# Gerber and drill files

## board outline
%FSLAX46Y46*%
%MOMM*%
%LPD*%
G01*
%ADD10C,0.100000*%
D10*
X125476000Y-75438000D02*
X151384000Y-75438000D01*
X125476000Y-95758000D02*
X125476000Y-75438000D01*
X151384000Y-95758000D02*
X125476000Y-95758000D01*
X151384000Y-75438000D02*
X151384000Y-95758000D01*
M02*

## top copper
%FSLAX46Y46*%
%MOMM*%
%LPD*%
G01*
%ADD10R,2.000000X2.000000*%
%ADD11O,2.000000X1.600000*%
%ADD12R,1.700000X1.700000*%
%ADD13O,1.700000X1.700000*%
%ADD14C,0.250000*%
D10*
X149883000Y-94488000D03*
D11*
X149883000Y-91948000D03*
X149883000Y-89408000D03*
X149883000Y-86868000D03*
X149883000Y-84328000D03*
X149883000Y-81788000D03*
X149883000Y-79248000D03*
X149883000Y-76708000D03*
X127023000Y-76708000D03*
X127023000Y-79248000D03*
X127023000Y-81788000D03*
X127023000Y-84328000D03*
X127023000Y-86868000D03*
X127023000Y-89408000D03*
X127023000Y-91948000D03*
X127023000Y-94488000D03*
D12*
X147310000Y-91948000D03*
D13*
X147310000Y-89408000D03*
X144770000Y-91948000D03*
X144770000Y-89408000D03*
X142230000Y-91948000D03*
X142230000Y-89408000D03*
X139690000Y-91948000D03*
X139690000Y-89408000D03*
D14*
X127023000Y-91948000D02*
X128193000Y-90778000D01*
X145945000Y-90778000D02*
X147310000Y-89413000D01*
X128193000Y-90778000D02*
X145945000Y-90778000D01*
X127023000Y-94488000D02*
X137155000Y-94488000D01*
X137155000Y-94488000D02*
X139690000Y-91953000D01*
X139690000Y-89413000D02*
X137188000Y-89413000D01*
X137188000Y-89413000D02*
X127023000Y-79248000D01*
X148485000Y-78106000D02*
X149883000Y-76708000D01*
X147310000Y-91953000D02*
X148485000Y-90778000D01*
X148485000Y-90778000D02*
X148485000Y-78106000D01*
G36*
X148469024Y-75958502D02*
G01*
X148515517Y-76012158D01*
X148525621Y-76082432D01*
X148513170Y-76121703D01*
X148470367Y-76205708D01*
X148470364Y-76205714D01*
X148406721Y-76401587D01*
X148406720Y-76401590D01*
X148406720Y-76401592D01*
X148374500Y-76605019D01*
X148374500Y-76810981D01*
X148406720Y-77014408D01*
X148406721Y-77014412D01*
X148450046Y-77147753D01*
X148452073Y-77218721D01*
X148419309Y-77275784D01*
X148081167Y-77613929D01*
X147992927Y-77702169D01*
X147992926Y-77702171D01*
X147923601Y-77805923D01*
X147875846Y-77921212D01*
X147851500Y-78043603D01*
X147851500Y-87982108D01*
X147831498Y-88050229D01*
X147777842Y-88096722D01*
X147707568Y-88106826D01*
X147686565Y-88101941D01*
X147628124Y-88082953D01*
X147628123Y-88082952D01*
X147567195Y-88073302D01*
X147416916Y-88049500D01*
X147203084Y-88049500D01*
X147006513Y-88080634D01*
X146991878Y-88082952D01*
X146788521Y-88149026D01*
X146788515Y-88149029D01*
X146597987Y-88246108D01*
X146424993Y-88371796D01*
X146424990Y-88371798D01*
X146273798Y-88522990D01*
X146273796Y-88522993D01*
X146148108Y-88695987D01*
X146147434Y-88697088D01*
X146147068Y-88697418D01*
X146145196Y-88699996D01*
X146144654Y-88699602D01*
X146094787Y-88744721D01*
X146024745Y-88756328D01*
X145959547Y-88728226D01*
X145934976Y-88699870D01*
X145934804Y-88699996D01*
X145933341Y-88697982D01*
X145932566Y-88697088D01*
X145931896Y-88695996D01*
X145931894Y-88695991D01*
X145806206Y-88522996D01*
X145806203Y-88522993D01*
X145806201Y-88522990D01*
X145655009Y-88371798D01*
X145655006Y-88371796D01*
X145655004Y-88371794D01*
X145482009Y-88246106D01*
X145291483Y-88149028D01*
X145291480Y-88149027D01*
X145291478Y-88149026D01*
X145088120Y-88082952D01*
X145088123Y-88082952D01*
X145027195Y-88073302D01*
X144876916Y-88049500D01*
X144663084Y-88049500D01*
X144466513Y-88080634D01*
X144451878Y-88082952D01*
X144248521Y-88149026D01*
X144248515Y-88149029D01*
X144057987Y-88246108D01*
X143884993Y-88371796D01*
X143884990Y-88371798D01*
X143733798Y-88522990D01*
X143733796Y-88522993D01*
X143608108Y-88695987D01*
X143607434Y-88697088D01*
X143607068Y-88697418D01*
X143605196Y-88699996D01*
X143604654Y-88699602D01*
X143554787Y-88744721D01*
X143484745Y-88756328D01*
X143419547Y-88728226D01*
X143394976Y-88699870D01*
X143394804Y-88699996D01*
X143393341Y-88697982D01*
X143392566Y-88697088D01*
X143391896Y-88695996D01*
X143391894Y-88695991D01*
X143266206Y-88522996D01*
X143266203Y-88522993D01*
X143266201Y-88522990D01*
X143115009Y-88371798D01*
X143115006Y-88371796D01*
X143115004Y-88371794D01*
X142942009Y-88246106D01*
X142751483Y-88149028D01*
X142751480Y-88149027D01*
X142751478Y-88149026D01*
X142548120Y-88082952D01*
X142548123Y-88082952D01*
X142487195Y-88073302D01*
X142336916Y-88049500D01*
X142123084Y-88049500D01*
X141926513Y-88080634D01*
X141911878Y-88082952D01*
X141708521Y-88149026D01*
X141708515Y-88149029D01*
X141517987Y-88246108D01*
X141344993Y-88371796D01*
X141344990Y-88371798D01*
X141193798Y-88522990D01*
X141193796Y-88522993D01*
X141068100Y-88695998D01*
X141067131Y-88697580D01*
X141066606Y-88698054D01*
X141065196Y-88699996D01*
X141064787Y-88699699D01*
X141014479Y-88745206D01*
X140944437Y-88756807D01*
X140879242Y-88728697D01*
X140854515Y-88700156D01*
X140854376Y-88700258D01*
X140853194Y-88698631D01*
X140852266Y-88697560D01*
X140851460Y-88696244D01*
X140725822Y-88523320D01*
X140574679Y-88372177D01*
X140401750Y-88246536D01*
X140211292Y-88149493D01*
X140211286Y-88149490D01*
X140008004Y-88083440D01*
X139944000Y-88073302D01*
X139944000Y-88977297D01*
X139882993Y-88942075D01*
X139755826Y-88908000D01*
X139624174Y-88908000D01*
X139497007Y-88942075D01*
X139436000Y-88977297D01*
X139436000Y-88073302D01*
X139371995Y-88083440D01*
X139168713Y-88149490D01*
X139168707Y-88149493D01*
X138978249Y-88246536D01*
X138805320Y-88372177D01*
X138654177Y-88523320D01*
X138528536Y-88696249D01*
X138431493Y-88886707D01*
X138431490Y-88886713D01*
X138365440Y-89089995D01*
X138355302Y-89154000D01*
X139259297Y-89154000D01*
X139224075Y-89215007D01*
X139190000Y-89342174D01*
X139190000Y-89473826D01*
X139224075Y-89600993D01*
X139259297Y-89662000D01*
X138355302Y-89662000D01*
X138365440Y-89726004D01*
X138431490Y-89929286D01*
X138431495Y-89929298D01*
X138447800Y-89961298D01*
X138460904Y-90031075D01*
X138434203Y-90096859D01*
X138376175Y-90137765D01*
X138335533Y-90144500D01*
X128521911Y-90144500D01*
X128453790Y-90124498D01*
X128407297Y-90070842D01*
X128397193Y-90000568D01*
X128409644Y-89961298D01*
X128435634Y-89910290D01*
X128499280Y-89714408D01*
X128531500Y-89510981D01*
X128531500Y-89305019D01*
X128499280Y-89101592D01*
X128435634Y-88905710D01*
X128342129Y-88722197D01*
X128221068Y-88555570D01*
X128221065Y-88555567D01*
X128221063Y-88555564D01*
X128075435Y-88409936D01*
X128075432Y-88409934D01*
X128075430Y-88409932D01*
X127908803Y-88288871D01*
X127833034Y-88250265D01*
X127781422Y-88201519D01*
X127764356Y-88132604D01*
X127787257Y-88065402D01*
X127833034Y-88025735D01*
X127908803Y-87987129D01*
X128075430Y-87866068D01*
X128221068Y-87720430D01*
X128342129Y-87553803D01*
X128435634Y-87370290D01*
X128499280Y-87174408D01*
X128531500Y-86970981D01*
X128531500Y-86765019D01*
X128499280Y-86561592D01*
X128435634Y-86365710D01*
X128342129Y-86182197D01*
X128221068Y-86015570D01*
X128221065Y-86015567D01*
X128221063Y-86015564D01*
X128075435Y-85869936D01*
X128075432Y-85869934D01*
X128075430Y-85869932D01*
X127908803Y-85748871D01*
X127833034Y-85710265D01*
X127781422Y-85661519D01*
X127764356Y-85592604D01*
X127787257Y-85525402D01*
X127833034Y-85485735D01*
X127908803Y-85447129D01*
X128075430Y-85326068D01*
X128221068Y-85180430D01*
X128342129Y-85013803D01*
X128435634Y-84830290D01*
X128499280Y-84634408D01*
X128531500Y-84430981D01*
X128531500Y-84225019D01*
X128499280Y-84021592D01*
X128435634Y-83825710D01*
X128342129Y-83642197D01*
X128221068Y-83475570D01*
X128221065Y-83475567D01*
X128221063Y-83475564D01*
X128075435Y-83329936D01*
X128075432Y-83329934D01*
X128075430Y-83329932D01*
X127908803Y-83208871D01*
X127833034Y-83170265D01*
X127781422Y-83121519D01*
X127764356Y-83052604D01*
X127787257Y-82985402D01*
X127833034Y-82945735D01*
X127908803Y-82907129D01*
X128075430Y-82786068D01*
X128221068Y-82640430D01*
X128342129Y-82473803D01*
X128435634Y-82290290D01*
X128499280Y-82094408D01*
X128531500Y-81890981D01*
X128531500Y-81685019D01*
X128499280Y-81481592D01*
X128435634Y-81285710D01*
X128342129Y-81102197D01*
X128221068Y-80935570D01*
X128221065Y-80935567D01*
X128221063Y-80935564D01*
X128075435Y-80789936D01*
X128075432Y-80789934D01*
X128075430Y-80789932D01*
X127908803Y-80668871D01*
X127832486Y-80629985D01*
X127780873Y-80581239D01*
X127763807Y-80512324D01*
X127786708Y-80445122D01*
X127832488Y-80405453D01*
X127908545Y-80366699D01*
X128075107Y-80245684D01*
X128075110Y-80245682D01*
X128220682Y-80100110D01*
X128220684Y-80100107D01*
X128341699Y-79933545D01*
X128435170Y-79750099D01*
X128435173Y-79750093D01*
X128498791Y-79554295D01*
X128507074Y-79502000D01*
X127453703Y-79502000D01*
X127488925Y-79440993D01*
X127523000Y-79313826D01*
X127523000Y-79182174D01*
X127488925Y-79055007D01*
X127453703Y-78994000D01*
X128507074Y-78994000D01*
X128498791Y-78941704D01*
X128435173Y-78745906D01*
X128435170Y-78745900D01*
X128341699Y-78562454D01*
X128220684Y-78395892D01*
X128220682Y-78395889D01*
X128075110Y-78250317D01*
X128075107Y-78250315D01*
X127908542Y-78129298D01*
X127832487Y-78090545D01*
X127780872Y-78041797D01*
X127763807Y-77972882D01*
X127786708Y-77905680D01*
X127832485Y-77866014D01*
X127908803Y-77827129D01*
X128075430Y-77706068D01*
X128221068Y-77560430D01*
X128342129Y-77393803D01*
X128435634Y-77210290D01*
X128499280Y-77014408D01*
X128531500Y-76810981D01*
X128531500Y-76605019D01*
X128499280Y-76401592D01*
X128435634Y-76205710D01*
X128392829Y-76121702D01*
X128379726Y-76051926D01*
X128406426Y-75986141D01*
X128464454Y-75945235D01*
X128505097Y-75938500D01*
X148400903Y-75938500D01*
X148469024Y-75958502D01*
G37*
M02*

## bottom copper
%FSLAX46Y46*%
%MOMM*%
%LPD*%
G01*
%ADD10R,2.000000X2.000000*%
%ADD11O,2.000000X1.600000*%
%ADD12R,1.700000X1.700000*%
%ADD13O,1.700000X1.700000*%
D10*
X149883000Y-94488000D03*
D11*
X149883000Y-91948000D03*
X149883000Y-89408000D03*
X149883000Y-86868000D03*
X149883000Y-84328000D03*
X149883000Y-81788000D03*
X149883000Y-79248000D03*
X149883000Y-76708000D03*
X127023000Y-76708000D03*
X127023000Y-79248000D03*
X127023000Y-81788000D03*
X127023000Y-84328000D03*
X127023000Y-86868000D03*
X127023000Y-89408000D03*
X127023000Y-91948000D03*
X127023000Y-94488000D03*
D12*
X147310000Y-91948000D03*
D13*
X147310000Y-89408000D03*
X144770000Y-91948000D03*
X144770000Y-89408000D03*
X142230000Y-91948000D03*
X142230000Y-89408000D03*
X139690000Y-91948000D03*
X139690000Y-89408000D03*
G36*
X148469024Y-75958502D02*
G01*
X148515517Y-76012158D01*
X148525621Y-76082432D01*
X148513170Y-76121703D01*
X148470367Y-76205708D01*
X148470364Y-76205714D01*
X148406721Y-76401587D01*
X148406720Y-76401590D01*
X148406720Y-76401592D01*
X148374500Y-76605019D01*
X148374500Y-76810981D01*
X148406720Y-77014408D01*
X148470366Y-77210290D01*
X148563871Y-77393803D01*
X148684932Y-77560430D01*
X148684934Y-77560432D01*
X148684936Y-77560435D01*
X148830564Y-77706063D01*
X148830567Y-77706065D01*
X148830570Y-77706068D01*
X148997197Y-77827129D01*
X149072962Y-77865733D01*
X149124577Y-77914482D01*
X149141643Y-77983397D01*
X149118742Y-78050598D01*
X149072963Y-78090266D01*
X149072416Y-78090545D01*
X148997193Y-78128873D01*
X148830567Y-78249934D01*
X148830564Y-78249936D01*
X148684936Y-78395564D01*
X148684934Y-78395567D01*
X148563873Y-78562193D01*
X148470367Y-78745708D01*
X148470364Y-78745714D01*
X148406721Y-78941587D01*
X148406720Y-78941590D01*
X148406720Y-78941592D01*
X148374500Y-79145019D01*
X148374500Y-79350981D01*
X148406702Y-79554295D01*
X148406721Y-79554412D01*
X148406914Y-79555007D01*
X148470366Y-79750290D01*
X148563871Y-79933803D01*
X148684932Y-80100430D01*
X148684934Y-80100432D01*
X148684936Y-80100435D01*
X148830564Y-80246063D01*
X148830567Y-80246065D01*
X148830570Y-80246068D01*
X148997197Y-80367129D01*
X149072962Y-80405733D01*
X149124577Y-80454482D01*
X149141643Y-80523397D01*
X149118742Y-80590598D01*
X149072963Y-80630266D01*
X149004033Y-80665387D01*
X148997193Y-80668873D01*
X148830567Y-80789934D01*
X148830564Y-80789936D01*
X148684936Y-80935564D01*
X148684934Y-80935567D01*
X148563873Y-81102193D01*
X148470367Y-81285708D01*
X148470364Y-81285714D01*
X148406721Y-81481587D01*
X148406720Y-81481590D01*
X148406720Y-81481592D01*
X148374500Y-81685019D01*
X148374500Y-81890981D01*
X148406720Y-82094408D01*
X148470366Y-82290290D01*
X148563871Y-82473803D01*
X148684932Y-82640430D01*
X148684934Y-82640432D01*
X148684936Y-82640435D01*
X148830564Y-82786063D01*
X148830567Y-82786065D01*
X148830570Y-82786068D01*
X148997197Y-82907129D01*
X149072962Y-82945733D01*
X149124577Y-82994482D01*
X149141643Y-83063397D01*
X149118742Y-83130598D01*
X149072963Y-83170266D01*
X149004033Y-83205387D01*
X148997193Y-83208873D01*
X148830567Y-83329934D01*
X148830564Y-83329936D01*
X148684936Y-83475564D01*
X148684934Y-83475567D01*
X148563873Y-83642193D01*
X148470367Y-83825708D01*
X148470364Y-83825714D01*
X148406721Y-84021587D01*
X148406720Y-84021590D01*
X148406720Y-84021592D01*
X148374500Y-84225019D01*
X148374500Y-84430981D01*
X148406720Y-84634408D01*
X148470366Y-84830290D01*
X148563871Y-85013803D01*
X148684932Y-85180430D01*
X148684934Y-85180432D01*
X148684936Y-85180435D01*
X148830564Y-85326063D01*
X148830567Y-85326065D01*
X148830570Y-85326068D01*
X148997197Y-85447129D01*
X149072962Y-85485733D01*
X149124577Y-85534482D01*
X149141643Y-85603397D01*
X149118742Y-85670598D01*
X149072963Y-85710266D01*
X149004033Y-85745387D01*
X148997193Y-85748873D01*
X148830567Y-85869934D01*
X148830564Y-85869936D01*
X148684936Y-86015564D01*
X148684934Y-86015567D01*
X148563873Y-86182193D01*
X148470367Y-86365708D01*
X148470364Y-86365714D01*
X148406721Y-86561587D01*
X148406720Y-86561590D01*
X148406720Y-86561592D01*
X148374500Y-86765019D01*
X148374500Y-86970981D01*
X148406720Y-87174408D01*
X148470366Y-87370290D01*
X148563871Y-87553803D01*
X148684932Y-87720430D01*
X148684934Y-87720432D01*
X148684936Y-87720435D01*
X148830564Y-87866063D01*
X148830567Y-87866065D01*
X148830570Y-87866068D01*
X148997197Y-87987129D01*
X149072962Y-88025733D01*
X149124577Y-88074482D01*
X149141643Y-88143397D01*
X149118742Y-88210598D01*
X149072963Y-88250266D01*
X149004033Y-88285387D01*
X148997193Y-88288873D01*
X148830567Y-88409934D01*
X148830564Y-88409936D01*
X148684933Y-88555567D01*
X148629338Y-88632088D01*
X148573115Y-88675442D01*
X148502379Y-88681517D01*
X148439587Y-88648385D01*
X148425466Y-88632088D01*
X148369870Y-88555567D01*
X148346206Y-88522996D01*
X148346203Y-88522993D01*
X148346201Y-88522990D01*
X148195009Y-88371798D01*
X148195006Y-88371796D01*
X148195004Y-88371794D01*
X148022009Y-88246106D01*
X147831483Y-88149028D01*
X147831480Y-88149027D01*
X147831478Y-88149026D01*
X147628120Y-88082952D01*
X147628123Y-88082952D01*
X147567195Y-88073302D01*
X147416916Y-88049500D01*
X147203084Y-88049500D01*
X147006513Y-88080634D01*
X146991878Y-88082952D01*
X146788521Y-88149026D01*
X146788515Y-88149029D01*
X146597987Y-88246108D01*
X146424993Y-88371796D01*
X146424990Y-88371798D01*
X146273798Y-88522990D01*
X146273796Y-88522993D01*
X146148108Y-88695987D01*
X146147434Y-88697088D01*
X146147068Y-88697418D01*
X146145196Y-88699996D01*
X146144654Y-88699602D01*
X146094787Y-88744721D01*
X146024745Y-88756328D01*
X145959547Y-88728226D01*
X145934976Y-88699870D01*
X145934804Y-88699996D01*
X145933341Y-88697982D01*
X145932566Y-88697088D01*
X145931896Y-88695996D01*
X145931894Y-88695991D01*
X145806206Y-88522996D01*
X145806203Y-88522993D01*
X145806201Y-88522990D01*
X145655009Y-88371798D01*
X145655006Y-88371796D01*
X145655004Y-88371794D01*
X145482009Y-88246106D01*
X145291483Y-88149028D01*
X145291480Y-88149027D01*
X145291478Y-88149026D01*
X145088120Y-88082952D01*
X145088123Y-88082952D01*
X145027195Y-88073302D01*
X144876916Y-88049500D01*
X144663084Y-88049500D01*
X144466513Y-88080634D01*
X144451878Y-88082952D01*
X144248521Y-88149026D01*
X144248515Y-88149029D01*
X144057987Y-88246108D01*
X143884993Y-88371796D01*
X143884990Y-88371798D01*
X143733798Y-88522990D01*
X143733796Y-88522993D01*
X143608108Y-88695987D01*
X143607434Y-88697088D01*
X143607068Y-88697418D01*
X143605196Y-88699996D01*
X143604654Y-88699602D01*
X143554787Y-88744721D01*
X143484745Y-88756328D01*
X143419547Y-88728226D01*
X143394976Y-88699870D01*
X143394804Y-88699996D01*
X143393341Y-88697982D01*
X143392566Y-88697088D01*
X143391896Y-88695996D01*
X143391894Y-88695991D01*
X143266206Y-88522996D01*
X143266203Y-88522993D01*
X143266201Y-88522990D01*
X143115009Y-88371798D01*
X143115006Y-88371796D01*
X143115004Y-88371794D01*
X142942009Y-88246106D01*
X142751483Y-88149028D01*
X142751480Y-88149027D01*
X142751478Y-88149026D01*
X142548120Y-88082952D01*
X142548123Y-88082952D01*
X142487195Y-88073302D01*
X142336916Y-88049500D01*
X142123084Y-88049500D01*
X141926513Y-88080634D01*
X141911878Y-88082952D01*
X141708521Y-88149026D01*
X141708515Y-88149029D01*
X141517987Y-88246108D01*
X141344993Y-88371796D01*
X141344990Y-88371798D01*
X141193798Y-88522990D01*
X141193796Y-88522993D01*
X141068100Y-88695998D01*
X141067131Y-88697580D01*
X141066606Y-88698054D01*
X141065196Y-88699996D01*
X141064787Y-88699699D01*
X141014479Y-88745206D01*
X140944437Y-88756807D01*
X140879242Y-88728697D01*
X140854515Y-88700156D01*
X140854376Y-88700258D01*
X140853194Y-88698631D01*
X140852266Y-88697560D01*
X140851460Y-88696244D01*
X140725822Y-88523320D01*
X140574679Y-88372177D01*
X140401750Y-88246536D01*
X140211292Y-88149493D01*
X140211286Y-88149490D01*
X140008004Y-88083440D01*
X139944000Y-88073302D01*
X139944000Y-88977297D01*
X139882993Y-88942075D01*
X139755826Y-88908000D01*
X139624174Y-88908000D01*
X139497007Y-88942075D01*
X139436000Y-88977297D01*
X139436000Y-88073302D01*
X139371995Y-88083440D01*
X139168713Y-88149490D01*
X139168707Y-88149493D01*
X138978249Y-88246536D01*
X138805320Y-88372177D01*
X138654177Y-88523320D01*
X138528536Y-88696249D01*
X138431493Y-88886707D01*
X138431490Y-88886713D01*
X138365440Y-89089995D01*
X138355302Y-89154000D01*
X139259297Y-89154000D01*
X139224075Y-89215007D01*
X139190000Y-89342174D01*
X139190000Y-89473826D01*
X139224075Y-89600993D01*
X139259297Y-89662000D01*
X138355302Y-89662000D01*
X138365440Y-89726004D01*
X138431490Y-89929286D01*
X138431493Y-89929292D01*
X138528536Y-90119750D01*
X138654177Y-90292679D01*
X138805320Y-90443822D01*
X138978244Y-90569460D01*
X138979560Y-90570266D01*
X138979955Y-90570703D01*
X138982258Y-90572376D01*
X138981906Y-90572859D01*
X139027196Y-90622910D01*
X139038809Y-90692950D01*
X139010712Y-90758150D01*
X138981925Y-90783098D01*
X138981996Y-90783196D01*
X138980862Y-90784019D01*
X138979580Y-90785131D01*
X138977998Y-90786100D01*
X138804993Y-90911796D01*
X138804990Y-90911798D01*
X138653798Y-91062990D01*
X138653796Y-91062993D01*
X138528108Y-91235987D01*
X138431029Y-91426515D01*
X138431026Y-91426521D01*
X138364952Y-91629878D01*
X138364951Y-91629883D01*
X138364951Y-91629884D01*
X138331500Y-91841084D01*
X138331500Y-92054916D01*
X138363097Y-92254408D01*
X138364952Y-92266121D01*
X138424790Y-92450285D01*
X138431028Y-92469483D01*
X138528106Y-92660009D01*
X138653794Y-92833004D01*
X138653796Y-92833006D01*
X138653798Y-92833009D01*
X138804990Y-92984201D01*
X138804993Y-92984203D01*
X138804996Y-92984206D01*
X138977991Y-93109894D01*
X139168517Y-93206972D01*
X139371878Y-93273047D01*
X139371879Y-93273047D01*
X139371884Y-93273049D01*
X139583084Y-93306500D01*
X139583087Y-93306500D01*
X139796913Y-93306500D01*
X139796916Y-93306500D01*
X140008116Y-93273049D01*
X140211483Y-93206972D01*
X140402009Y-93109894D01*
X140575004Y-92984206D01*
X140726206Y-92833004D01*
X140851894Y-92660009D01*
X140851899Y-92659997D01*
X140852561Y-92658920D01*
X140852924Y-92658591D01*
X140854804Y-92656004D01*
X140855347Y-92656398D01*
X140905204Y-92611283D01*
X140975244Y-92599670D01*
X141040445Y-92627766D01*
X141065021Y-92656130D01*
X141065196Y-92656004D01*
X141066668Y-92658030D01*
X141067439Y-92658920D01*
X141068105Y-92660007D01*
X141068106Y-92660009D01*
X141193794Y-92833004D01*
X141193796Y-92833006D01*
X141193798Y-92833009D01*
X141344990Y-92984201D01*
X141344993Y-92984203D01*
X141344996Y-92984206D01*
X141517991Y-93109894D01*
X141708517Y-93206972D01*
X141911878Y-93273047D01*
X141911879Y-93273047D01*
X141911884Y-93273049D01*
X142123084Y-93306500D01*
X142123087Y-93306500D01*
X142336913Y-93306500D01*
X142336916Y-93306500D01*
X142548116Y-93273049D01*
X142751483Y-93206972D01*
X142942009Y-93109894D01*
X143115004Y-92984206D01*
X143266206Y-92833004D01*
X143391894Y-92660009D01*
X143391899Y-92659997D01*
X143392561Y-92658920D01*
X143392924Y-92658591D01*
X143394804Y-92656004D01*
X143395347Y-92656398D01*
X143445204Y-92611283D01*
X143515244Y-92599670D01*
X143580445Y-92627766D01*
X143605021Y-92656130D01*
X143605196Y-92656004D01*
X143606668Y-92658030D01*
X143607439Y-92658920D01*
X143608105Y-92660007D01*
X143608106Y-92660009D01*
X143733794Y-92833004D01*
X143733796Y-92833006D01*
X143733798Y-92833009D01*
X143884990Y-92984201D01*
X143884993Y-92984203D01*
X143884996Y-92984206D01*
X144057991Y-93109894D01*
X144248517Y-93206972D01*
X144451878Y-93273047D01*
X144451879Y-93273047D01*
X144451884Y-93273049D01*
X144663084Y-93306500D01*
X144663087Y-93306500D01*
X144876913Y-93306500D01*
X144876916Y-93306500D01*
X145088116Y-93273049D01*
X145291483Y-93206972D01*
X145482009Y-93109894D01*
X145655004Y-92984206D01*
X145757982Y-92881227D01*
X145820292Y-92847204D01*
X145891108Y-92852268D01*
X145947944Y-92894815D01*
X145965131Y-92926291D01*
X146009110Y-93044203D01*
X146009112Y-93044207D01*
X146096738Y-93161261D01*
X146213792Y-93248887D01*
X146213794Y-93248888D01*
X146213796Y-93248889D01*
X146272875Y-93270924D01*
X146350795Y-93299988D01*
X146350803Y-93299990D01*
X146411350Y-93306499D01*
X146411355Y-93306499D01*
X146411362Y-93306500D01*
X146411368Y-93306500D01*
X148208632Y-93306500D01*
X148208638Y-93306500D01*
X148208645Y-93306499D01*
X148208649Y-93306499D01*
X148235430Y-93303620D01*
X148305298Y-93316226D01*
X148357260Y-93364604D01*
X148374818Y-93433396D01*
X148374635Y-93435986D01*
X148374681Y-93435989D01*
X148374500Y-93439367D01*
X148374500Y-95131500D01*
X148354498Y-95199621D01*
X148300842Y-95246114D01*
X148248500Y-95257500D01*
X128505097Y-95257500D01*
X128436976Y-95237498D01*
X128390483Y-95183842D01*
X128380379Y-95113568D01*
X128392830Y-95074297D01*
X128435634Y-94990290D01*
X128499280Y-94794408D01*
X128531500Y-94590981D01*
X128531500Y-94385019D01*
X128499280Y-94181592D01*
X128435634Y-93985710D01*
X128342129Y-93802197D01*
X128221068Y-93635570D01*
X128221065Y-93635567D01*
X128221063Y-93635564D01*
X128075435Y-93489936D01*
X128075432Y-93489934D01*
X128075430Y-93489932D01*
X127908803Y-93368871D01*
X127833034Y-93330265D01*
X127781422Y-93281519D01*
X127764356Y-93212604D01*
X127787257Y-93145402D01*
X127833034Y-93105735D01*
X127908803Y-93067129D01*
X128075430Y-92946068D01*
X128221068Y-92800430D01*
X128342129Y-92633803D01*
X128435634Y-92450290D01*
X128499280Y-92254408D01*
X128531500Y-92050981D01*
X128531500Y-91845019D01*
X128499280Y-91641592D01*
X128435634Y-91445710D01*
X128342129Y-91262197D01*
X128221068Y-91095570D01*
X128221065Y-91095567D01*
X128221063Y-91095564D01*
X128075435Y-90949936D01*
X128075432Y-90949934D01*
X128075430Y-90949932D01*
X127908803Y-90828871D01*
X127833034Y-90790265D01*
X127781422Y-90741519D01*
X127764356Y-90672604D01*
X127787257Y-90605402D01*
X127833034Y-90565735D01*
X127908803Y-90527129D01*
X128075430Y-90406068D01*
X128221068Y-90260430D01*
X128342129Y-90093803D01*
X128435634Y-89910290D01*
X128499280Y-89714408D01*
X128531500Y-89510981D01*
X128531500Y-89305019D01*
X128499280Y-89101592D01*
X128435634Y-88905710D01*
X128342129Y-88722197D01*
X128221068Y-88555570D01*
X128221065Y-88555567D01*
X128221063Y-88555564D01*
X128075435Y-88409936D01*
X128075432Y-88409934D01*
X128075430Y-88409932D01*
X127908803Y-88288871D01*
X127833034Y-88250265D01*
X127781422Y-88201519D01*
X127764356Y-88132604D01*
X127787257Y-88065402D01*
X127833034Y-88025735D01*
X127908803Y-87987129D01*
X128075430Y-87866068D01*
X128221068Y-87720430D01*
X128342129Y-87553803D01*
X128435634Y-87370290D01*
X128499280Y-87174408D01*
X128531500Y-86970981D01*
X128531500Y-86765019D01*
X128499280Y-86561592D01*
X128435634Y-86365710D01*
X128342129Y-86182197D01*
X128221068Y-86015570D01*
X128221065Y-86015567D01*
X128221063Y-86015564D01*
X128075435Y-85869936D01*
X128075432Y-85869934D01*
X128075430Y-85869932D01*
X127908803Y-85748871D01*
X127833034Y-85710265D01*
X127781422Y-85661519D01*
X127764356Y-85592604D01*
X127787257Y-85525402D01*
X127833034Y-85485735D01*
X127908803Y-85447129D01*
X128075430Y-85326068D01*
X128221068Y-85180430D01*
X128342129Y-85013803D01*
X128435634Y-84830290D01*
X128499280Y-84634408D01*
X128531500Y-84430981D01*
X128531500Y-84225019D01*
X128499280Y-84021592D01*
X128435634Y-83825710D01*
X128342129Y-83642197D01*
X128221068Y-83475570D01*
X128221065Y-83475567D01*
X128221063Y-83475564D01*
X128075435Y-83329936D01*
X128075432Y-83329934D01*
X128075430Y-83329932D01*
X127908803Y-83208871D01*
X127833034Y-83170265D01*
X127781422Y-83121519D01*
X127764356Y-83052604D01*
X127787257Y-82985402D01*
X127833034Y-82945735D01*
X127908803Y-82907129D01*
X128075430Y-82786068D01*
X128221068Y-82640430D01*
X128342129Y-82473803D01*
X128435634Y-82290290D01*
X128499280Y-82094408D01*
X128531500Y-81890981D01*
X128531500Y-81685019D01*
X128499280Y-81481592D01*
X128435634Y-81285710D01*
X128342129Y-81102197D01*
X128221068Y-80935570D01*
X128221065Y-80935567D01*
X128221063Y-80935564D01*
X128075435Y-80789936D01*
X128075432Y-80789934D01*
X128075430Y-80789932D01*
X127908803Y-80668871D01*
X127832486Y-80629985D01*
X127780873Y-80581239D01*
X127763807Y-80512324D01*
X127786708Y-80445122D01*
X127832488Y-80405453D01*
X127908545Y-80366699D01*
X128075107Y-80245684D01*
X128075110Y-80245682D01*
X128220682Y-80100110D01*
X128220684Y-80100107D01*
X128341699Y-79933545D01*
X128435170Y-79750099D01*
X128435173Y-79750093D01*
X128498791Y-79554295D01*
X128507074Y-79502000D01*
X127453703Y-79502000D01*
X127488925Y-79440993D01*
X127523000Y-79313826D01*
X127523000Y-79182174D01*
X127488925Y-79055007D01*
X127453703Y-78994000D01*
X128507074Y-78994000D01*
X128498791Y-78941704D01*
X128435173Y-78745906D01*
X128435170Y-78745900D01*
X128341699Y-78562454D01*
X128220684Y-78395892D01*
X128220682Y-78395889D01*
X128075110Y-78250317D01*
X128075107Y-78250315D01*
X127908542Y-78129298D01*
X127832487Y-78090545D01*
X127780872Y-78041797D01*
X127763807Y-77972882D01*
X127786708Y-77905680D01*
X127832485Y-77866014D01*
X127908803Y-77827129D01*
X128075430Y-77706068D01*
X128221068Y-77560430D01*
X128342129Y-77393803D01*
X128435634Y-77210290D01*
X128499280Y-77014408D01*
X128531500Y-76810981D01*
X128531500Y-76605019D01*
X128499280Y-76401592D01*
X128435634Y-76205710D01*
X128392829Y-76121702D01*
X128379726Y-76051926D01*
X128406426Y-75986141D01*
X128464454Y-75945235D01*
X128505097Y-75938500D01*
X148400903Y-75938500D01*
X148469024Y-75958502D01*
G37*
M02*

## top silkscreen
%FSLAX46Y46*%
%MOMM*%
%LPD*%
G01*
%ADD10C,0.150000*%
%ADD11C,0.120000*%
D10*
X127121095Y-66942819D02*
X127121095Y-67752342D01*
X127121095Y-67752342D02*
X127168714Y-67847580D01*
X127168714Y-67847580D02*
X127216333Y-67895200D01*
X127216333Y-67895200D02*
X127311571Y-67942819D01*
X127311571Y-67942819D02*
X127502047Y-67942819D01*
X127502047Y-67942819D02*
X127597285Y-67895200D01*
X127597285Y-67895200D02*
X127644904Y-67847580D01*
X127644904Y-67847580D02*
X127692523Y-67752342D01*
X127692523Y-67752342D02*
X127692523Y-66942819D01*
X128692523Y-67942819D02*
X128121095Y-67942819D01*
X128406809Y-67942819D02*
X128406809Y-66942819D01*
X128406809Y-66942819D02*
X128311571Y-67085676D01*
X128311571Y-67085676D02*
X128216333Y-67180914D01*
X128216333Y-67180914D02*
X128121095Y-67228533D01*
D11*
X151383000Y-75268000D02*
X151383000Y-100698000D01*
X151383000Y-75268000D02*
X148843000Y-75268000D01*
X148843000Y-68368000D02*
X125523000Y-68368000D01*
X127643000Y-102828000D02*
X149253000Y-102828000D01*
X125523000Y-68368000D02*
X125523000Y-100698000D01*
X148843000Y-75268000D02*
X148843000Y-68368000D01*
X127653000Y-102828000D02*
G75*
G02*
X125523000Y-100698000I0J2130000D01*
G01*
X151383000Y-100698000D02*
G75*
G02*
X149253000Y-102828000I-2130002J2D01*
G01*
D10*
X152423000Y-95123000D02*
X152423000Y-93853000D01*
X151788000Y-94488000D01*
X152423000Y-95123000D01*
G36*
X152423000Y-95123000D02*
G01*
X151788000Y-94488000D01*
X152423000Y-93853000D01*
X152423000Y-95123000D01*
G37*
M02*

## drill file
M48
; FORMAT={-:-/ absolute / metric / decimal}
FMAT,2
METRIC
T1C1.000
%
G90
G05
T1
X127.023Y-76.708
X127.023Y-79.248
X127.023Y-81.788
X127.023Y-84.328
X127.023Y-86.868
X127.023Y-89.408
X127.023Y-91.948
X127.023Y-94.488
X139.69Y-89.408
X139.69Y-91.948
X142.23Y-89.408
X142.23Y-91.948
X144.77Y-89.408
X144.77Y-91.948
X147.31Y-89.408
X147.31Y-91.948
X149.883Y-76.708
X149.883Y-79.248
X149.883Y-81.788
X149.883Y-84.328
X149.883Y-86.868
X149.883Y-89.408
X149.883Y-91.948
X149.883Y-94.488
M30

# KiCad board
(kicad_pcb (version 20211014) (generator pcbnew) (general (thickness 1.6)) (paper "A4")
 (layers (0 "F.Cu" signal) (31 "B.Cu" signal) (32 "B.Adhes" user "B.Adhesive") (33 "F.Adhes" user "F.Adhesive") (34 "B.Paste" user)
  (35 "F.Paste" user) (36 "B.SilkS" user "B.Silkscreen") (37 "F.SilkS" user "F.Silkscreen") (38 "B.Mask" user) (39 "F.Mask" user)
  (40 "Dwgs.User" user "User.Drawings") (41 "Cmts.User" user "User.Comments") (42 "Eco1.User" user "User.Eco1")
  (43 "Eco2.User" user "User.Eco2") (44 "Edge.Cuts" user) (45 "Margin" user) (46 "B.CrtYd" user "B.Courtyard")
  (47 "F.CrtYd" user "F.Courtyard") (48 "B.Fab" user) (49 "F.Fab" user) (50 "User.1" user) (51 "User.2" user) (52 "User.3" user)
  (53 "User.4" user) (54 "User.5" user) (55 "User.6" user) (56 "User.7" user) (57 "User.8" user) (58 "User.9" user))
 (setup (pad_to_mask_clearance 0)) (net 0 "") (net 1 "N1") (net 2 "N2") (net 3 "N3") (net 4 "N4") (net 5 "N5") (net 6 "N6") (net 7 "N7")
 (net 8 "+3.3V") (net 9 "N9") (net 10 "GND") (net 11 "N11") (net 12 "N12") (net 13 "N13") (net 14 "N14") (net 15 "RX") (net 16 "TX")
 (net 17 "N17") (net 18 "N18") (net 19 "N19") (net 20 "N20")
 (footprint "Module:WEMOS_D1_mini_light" (layer "F.Cu") (at 149.883 94.488 180)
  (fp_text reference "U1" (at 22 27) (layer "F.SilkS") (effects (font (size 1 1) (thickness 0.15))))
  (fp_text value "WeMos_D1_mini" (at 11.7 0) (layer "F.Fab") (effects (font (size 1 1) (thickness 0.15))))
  (fp_line (start -1.5 19.22) (end -1.5 -6.21) (layer "F.SilkS") (width 0.12))
  (fp_line (start -1.5 19.22) (end 1.04 19.22) (layer "F.SilkS") (width 0.12))
  (fp_line (start 1.04 26.12) (end 24.36 26.12) (layer "F.SilkS") (width 0.12))
  (fp_line (start 22.24 -8.34) (end 0.63 -8.34) (layer "F.SilkS") (width 0.12))
  (fp_line (start 24.36 26.12) (end 24.36 -6.21) (layer "F.SilkS") (width 0.12))
  (fp_line (start 1.04 19.22) (end 1.04 26.12) (layer "F.SilkS") (width 0.12))
  (fp_arc (start 22.23 -8.34) (mid 23.736137 -7.716137) (end 24.36 -6.21) (layer "F.SilkS") (width 0.12))
  (fp_arc (start -1.5 -6.21) (mid -0.876137 -7.716137) (end 0.63 -8.34) (layer "F.SilkS") (width 0.12))
  (fp_poly (pts (xy -2.54 -0.635) (xy -2.54 0.635) (xy -1.905 0)) (layer "F.SilkS") (width 0.15) (fill solid))
  (pad "1" thru_hole rect (at 0 0 180) (size 2 2) (drill 1) (layers *.Cu *.Mask) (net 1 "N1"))
  (pad "2" thru_hole oval (at 0 2.54 180) (size 2 1.6) (drill 1) (layers *.Cu *.Mask) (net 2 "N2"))
  (pad "3" thru_hole oval (at 0 5.08 180) (size 2 1.6) (drill 1) (layers *.Cu *.Mask) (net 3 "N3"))
  (pad "4" thru_hole oval (at 0 7.62 180) (size 2 1.6) (drill 1) (layers *.Cu *.Mask) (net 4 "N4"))
  (pad "5" thru_hole oval (at 0 10.16 180) (size 2 1.6) (drill 1) (layers *.Cu *.Mask) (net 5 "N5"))
  (pad "6" thru_hole oval (at 0 12.7 180) (size 2 1.6) (drill 1) (layers *.Cu *.Mask) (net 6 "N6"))
  (pad "7" thru_hole oval (at 0 15.24 180) (size 2 1.6) (drill 1) (layers *.Cu *.Mask) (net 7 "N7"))
  (pad "8" thru_hole oval (at 0 17.78 180) (size 2 1.6) (drill 1) (layers *.Cu *.Mask) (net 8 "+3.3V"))
  (pad "9" thru_hole oval (at 22.86 17.78 180) (size 2 1.6) (drill 1) (layers *.Cu *.Mask) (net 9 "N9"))
  (pad "10" thru_hole oval (at 22.86 15.24 180) (size 2 1.6) (drill 1) (layers *.Cu *.Mask) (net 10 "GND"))
  (pad "11" thru_hole oval (at 22.86 12.7 180) (size 2 1.6) (drill 1) (layers *.Cu *.Mask) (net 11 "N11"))
  (pad "12" thru_hole oval (at 22.86 10.16 180) (size 2 1.6) (drill 1) (layers *.Cu *.Mask) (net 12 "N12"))
  (pad "13" thru_hole oval (at 22.86 7.62 180) (size 2 1.6) (drill 1) (layers *.Cu *.Mask) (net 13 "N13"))
  (pad "14" thru_hole oval (at 22.86 5.08 180) (size 2 1.6) (drill 1) (layers *.Cu *.Mask) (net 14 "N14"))
  (pad "15" thru_hole oval (at 22.86 2.54 180) (size 2 1.6) (drill 1) (layers *.Cu *.Mask) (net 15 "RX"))
  (pad "16" thru_hole oval (at 22.86 0 180) (size 2 1.6) (drill 1) (layers *.Cu *.Mask) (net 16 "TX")))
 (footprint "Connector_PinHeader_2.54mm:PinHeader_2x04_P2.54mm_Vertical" (layer "B.Cu") (at 147.31 91.948 90)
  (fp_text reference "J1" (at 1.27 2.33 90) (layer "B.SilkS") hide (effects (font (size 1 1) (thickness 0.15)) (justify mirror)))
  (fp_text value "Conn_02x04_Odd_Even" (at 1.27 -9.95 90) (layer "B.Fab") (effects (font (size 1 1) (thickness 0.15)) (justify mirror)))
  (pad "1" thru_hole rect (at 0 0 90) (size 1.7 1.7) (drill 1) (layers *.Cu *.Mask) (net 8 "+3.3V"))
  (pad "2" thru_hole oval (at 2.54 0 90) (size 1.7 1.7) (drill 1) (layers *.Cu *.Mask) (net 15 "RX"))
  (pad "3" thru_hole oval (at 0 -2.54 90) (size 1.7 1.7) (drill 1) (layers *.Cu *.Mask) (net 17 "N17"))
  (pad "4" thru_hole oval (at 2.54 -2.54 90) (size 1.7 1.7) (drill 1) (layers *.Cu *.Mask) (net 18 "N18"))
  (pad "5" thru_hole oval (at 0 -5.08 90) (size 1.7 1.7) (drill 1) (layers *.Cu *.Mask) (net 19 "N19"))
  (pad "6" thru_hole oval (at 2.54 -5.08 90) (size 1.7 1.7) (drill 1) (layers *.Cu *.Mask) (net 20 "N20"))
  (pad "7" thru_hole oval (at 0 -7.62 90) (size 1.7 1.7) (drill 1) (layers *.Cu *.Mask) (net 16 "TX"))
  (pad "8" thru_hole oval (at 2.54 -7.62 90) (size 1.7 1.7) (drill 1) (layers *.Cu *.Mask) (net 10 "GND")))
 (gr_line (start 125.476 75.438) (end 151.384 75.438) (layer "Edge.Cuts") (width 0.1))
 (gr_line (start 125.476 95.758) (end 125.476 75.438) (layer "Edge.Cuts") (width 0.1))
 (gr_line (start 151.384 95.758) (end 125.476 95.758) (layer "Edge.Cuts") (width 0.1))
 (gr_line (start 151.384 75.438) (end 151.384 95.758) (layer "Edge.Cuts") (width 0.1))
 (segment (start 127.023 91.948) (end 128.193 90.778) (width 0.25) (layer "F.Cu") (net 15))
 (segment (start 145.945 90.778) (end 147.31 89.413) (width 0.25) (layer "F.Cu") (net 15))
 (segment (start 128.193 90.778) (end 145.945 90.778) (width 0.25) (layer "F.Cu") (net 15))
 (segment (start 127.023 94.488) (end 137.155 94.488) (width 0.25) (layer "F.Cu") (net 16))
 (segment (start 137.155 94.488) (end 139.69 91.953) (width 0.25) (layer "F.Cu") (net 16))
 (segment (start 139.69 89.413) (end 137.188 89.413) (width 0.25) (layer "F.Cu") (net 10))
 (segment (start 137.188 89.413) (end 127.023 79.248) (width 0.25) (layer "F.Cu") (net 10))
 (segment (start 148.485 78.106) (end 149.883 76.708) (width 0.25) (layer "F.Cu") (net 8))
 (segment (start 147.31 91.953) (end 148.485 90.778) (width 0.25) (layer "F.Cu") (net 8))
 (segment (start 148.485 90.778) (end 148.485 78.106) (width 0.25) (layer "F.Cu") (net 8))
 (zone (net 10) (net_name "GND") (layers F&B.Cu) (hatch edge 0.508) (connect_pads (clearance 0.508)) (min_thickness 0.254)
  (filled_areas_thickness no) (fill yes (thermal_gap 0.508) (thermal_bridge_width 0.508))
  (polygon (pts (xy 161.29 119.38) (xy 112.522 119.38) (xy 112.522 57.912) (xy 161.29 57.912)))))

